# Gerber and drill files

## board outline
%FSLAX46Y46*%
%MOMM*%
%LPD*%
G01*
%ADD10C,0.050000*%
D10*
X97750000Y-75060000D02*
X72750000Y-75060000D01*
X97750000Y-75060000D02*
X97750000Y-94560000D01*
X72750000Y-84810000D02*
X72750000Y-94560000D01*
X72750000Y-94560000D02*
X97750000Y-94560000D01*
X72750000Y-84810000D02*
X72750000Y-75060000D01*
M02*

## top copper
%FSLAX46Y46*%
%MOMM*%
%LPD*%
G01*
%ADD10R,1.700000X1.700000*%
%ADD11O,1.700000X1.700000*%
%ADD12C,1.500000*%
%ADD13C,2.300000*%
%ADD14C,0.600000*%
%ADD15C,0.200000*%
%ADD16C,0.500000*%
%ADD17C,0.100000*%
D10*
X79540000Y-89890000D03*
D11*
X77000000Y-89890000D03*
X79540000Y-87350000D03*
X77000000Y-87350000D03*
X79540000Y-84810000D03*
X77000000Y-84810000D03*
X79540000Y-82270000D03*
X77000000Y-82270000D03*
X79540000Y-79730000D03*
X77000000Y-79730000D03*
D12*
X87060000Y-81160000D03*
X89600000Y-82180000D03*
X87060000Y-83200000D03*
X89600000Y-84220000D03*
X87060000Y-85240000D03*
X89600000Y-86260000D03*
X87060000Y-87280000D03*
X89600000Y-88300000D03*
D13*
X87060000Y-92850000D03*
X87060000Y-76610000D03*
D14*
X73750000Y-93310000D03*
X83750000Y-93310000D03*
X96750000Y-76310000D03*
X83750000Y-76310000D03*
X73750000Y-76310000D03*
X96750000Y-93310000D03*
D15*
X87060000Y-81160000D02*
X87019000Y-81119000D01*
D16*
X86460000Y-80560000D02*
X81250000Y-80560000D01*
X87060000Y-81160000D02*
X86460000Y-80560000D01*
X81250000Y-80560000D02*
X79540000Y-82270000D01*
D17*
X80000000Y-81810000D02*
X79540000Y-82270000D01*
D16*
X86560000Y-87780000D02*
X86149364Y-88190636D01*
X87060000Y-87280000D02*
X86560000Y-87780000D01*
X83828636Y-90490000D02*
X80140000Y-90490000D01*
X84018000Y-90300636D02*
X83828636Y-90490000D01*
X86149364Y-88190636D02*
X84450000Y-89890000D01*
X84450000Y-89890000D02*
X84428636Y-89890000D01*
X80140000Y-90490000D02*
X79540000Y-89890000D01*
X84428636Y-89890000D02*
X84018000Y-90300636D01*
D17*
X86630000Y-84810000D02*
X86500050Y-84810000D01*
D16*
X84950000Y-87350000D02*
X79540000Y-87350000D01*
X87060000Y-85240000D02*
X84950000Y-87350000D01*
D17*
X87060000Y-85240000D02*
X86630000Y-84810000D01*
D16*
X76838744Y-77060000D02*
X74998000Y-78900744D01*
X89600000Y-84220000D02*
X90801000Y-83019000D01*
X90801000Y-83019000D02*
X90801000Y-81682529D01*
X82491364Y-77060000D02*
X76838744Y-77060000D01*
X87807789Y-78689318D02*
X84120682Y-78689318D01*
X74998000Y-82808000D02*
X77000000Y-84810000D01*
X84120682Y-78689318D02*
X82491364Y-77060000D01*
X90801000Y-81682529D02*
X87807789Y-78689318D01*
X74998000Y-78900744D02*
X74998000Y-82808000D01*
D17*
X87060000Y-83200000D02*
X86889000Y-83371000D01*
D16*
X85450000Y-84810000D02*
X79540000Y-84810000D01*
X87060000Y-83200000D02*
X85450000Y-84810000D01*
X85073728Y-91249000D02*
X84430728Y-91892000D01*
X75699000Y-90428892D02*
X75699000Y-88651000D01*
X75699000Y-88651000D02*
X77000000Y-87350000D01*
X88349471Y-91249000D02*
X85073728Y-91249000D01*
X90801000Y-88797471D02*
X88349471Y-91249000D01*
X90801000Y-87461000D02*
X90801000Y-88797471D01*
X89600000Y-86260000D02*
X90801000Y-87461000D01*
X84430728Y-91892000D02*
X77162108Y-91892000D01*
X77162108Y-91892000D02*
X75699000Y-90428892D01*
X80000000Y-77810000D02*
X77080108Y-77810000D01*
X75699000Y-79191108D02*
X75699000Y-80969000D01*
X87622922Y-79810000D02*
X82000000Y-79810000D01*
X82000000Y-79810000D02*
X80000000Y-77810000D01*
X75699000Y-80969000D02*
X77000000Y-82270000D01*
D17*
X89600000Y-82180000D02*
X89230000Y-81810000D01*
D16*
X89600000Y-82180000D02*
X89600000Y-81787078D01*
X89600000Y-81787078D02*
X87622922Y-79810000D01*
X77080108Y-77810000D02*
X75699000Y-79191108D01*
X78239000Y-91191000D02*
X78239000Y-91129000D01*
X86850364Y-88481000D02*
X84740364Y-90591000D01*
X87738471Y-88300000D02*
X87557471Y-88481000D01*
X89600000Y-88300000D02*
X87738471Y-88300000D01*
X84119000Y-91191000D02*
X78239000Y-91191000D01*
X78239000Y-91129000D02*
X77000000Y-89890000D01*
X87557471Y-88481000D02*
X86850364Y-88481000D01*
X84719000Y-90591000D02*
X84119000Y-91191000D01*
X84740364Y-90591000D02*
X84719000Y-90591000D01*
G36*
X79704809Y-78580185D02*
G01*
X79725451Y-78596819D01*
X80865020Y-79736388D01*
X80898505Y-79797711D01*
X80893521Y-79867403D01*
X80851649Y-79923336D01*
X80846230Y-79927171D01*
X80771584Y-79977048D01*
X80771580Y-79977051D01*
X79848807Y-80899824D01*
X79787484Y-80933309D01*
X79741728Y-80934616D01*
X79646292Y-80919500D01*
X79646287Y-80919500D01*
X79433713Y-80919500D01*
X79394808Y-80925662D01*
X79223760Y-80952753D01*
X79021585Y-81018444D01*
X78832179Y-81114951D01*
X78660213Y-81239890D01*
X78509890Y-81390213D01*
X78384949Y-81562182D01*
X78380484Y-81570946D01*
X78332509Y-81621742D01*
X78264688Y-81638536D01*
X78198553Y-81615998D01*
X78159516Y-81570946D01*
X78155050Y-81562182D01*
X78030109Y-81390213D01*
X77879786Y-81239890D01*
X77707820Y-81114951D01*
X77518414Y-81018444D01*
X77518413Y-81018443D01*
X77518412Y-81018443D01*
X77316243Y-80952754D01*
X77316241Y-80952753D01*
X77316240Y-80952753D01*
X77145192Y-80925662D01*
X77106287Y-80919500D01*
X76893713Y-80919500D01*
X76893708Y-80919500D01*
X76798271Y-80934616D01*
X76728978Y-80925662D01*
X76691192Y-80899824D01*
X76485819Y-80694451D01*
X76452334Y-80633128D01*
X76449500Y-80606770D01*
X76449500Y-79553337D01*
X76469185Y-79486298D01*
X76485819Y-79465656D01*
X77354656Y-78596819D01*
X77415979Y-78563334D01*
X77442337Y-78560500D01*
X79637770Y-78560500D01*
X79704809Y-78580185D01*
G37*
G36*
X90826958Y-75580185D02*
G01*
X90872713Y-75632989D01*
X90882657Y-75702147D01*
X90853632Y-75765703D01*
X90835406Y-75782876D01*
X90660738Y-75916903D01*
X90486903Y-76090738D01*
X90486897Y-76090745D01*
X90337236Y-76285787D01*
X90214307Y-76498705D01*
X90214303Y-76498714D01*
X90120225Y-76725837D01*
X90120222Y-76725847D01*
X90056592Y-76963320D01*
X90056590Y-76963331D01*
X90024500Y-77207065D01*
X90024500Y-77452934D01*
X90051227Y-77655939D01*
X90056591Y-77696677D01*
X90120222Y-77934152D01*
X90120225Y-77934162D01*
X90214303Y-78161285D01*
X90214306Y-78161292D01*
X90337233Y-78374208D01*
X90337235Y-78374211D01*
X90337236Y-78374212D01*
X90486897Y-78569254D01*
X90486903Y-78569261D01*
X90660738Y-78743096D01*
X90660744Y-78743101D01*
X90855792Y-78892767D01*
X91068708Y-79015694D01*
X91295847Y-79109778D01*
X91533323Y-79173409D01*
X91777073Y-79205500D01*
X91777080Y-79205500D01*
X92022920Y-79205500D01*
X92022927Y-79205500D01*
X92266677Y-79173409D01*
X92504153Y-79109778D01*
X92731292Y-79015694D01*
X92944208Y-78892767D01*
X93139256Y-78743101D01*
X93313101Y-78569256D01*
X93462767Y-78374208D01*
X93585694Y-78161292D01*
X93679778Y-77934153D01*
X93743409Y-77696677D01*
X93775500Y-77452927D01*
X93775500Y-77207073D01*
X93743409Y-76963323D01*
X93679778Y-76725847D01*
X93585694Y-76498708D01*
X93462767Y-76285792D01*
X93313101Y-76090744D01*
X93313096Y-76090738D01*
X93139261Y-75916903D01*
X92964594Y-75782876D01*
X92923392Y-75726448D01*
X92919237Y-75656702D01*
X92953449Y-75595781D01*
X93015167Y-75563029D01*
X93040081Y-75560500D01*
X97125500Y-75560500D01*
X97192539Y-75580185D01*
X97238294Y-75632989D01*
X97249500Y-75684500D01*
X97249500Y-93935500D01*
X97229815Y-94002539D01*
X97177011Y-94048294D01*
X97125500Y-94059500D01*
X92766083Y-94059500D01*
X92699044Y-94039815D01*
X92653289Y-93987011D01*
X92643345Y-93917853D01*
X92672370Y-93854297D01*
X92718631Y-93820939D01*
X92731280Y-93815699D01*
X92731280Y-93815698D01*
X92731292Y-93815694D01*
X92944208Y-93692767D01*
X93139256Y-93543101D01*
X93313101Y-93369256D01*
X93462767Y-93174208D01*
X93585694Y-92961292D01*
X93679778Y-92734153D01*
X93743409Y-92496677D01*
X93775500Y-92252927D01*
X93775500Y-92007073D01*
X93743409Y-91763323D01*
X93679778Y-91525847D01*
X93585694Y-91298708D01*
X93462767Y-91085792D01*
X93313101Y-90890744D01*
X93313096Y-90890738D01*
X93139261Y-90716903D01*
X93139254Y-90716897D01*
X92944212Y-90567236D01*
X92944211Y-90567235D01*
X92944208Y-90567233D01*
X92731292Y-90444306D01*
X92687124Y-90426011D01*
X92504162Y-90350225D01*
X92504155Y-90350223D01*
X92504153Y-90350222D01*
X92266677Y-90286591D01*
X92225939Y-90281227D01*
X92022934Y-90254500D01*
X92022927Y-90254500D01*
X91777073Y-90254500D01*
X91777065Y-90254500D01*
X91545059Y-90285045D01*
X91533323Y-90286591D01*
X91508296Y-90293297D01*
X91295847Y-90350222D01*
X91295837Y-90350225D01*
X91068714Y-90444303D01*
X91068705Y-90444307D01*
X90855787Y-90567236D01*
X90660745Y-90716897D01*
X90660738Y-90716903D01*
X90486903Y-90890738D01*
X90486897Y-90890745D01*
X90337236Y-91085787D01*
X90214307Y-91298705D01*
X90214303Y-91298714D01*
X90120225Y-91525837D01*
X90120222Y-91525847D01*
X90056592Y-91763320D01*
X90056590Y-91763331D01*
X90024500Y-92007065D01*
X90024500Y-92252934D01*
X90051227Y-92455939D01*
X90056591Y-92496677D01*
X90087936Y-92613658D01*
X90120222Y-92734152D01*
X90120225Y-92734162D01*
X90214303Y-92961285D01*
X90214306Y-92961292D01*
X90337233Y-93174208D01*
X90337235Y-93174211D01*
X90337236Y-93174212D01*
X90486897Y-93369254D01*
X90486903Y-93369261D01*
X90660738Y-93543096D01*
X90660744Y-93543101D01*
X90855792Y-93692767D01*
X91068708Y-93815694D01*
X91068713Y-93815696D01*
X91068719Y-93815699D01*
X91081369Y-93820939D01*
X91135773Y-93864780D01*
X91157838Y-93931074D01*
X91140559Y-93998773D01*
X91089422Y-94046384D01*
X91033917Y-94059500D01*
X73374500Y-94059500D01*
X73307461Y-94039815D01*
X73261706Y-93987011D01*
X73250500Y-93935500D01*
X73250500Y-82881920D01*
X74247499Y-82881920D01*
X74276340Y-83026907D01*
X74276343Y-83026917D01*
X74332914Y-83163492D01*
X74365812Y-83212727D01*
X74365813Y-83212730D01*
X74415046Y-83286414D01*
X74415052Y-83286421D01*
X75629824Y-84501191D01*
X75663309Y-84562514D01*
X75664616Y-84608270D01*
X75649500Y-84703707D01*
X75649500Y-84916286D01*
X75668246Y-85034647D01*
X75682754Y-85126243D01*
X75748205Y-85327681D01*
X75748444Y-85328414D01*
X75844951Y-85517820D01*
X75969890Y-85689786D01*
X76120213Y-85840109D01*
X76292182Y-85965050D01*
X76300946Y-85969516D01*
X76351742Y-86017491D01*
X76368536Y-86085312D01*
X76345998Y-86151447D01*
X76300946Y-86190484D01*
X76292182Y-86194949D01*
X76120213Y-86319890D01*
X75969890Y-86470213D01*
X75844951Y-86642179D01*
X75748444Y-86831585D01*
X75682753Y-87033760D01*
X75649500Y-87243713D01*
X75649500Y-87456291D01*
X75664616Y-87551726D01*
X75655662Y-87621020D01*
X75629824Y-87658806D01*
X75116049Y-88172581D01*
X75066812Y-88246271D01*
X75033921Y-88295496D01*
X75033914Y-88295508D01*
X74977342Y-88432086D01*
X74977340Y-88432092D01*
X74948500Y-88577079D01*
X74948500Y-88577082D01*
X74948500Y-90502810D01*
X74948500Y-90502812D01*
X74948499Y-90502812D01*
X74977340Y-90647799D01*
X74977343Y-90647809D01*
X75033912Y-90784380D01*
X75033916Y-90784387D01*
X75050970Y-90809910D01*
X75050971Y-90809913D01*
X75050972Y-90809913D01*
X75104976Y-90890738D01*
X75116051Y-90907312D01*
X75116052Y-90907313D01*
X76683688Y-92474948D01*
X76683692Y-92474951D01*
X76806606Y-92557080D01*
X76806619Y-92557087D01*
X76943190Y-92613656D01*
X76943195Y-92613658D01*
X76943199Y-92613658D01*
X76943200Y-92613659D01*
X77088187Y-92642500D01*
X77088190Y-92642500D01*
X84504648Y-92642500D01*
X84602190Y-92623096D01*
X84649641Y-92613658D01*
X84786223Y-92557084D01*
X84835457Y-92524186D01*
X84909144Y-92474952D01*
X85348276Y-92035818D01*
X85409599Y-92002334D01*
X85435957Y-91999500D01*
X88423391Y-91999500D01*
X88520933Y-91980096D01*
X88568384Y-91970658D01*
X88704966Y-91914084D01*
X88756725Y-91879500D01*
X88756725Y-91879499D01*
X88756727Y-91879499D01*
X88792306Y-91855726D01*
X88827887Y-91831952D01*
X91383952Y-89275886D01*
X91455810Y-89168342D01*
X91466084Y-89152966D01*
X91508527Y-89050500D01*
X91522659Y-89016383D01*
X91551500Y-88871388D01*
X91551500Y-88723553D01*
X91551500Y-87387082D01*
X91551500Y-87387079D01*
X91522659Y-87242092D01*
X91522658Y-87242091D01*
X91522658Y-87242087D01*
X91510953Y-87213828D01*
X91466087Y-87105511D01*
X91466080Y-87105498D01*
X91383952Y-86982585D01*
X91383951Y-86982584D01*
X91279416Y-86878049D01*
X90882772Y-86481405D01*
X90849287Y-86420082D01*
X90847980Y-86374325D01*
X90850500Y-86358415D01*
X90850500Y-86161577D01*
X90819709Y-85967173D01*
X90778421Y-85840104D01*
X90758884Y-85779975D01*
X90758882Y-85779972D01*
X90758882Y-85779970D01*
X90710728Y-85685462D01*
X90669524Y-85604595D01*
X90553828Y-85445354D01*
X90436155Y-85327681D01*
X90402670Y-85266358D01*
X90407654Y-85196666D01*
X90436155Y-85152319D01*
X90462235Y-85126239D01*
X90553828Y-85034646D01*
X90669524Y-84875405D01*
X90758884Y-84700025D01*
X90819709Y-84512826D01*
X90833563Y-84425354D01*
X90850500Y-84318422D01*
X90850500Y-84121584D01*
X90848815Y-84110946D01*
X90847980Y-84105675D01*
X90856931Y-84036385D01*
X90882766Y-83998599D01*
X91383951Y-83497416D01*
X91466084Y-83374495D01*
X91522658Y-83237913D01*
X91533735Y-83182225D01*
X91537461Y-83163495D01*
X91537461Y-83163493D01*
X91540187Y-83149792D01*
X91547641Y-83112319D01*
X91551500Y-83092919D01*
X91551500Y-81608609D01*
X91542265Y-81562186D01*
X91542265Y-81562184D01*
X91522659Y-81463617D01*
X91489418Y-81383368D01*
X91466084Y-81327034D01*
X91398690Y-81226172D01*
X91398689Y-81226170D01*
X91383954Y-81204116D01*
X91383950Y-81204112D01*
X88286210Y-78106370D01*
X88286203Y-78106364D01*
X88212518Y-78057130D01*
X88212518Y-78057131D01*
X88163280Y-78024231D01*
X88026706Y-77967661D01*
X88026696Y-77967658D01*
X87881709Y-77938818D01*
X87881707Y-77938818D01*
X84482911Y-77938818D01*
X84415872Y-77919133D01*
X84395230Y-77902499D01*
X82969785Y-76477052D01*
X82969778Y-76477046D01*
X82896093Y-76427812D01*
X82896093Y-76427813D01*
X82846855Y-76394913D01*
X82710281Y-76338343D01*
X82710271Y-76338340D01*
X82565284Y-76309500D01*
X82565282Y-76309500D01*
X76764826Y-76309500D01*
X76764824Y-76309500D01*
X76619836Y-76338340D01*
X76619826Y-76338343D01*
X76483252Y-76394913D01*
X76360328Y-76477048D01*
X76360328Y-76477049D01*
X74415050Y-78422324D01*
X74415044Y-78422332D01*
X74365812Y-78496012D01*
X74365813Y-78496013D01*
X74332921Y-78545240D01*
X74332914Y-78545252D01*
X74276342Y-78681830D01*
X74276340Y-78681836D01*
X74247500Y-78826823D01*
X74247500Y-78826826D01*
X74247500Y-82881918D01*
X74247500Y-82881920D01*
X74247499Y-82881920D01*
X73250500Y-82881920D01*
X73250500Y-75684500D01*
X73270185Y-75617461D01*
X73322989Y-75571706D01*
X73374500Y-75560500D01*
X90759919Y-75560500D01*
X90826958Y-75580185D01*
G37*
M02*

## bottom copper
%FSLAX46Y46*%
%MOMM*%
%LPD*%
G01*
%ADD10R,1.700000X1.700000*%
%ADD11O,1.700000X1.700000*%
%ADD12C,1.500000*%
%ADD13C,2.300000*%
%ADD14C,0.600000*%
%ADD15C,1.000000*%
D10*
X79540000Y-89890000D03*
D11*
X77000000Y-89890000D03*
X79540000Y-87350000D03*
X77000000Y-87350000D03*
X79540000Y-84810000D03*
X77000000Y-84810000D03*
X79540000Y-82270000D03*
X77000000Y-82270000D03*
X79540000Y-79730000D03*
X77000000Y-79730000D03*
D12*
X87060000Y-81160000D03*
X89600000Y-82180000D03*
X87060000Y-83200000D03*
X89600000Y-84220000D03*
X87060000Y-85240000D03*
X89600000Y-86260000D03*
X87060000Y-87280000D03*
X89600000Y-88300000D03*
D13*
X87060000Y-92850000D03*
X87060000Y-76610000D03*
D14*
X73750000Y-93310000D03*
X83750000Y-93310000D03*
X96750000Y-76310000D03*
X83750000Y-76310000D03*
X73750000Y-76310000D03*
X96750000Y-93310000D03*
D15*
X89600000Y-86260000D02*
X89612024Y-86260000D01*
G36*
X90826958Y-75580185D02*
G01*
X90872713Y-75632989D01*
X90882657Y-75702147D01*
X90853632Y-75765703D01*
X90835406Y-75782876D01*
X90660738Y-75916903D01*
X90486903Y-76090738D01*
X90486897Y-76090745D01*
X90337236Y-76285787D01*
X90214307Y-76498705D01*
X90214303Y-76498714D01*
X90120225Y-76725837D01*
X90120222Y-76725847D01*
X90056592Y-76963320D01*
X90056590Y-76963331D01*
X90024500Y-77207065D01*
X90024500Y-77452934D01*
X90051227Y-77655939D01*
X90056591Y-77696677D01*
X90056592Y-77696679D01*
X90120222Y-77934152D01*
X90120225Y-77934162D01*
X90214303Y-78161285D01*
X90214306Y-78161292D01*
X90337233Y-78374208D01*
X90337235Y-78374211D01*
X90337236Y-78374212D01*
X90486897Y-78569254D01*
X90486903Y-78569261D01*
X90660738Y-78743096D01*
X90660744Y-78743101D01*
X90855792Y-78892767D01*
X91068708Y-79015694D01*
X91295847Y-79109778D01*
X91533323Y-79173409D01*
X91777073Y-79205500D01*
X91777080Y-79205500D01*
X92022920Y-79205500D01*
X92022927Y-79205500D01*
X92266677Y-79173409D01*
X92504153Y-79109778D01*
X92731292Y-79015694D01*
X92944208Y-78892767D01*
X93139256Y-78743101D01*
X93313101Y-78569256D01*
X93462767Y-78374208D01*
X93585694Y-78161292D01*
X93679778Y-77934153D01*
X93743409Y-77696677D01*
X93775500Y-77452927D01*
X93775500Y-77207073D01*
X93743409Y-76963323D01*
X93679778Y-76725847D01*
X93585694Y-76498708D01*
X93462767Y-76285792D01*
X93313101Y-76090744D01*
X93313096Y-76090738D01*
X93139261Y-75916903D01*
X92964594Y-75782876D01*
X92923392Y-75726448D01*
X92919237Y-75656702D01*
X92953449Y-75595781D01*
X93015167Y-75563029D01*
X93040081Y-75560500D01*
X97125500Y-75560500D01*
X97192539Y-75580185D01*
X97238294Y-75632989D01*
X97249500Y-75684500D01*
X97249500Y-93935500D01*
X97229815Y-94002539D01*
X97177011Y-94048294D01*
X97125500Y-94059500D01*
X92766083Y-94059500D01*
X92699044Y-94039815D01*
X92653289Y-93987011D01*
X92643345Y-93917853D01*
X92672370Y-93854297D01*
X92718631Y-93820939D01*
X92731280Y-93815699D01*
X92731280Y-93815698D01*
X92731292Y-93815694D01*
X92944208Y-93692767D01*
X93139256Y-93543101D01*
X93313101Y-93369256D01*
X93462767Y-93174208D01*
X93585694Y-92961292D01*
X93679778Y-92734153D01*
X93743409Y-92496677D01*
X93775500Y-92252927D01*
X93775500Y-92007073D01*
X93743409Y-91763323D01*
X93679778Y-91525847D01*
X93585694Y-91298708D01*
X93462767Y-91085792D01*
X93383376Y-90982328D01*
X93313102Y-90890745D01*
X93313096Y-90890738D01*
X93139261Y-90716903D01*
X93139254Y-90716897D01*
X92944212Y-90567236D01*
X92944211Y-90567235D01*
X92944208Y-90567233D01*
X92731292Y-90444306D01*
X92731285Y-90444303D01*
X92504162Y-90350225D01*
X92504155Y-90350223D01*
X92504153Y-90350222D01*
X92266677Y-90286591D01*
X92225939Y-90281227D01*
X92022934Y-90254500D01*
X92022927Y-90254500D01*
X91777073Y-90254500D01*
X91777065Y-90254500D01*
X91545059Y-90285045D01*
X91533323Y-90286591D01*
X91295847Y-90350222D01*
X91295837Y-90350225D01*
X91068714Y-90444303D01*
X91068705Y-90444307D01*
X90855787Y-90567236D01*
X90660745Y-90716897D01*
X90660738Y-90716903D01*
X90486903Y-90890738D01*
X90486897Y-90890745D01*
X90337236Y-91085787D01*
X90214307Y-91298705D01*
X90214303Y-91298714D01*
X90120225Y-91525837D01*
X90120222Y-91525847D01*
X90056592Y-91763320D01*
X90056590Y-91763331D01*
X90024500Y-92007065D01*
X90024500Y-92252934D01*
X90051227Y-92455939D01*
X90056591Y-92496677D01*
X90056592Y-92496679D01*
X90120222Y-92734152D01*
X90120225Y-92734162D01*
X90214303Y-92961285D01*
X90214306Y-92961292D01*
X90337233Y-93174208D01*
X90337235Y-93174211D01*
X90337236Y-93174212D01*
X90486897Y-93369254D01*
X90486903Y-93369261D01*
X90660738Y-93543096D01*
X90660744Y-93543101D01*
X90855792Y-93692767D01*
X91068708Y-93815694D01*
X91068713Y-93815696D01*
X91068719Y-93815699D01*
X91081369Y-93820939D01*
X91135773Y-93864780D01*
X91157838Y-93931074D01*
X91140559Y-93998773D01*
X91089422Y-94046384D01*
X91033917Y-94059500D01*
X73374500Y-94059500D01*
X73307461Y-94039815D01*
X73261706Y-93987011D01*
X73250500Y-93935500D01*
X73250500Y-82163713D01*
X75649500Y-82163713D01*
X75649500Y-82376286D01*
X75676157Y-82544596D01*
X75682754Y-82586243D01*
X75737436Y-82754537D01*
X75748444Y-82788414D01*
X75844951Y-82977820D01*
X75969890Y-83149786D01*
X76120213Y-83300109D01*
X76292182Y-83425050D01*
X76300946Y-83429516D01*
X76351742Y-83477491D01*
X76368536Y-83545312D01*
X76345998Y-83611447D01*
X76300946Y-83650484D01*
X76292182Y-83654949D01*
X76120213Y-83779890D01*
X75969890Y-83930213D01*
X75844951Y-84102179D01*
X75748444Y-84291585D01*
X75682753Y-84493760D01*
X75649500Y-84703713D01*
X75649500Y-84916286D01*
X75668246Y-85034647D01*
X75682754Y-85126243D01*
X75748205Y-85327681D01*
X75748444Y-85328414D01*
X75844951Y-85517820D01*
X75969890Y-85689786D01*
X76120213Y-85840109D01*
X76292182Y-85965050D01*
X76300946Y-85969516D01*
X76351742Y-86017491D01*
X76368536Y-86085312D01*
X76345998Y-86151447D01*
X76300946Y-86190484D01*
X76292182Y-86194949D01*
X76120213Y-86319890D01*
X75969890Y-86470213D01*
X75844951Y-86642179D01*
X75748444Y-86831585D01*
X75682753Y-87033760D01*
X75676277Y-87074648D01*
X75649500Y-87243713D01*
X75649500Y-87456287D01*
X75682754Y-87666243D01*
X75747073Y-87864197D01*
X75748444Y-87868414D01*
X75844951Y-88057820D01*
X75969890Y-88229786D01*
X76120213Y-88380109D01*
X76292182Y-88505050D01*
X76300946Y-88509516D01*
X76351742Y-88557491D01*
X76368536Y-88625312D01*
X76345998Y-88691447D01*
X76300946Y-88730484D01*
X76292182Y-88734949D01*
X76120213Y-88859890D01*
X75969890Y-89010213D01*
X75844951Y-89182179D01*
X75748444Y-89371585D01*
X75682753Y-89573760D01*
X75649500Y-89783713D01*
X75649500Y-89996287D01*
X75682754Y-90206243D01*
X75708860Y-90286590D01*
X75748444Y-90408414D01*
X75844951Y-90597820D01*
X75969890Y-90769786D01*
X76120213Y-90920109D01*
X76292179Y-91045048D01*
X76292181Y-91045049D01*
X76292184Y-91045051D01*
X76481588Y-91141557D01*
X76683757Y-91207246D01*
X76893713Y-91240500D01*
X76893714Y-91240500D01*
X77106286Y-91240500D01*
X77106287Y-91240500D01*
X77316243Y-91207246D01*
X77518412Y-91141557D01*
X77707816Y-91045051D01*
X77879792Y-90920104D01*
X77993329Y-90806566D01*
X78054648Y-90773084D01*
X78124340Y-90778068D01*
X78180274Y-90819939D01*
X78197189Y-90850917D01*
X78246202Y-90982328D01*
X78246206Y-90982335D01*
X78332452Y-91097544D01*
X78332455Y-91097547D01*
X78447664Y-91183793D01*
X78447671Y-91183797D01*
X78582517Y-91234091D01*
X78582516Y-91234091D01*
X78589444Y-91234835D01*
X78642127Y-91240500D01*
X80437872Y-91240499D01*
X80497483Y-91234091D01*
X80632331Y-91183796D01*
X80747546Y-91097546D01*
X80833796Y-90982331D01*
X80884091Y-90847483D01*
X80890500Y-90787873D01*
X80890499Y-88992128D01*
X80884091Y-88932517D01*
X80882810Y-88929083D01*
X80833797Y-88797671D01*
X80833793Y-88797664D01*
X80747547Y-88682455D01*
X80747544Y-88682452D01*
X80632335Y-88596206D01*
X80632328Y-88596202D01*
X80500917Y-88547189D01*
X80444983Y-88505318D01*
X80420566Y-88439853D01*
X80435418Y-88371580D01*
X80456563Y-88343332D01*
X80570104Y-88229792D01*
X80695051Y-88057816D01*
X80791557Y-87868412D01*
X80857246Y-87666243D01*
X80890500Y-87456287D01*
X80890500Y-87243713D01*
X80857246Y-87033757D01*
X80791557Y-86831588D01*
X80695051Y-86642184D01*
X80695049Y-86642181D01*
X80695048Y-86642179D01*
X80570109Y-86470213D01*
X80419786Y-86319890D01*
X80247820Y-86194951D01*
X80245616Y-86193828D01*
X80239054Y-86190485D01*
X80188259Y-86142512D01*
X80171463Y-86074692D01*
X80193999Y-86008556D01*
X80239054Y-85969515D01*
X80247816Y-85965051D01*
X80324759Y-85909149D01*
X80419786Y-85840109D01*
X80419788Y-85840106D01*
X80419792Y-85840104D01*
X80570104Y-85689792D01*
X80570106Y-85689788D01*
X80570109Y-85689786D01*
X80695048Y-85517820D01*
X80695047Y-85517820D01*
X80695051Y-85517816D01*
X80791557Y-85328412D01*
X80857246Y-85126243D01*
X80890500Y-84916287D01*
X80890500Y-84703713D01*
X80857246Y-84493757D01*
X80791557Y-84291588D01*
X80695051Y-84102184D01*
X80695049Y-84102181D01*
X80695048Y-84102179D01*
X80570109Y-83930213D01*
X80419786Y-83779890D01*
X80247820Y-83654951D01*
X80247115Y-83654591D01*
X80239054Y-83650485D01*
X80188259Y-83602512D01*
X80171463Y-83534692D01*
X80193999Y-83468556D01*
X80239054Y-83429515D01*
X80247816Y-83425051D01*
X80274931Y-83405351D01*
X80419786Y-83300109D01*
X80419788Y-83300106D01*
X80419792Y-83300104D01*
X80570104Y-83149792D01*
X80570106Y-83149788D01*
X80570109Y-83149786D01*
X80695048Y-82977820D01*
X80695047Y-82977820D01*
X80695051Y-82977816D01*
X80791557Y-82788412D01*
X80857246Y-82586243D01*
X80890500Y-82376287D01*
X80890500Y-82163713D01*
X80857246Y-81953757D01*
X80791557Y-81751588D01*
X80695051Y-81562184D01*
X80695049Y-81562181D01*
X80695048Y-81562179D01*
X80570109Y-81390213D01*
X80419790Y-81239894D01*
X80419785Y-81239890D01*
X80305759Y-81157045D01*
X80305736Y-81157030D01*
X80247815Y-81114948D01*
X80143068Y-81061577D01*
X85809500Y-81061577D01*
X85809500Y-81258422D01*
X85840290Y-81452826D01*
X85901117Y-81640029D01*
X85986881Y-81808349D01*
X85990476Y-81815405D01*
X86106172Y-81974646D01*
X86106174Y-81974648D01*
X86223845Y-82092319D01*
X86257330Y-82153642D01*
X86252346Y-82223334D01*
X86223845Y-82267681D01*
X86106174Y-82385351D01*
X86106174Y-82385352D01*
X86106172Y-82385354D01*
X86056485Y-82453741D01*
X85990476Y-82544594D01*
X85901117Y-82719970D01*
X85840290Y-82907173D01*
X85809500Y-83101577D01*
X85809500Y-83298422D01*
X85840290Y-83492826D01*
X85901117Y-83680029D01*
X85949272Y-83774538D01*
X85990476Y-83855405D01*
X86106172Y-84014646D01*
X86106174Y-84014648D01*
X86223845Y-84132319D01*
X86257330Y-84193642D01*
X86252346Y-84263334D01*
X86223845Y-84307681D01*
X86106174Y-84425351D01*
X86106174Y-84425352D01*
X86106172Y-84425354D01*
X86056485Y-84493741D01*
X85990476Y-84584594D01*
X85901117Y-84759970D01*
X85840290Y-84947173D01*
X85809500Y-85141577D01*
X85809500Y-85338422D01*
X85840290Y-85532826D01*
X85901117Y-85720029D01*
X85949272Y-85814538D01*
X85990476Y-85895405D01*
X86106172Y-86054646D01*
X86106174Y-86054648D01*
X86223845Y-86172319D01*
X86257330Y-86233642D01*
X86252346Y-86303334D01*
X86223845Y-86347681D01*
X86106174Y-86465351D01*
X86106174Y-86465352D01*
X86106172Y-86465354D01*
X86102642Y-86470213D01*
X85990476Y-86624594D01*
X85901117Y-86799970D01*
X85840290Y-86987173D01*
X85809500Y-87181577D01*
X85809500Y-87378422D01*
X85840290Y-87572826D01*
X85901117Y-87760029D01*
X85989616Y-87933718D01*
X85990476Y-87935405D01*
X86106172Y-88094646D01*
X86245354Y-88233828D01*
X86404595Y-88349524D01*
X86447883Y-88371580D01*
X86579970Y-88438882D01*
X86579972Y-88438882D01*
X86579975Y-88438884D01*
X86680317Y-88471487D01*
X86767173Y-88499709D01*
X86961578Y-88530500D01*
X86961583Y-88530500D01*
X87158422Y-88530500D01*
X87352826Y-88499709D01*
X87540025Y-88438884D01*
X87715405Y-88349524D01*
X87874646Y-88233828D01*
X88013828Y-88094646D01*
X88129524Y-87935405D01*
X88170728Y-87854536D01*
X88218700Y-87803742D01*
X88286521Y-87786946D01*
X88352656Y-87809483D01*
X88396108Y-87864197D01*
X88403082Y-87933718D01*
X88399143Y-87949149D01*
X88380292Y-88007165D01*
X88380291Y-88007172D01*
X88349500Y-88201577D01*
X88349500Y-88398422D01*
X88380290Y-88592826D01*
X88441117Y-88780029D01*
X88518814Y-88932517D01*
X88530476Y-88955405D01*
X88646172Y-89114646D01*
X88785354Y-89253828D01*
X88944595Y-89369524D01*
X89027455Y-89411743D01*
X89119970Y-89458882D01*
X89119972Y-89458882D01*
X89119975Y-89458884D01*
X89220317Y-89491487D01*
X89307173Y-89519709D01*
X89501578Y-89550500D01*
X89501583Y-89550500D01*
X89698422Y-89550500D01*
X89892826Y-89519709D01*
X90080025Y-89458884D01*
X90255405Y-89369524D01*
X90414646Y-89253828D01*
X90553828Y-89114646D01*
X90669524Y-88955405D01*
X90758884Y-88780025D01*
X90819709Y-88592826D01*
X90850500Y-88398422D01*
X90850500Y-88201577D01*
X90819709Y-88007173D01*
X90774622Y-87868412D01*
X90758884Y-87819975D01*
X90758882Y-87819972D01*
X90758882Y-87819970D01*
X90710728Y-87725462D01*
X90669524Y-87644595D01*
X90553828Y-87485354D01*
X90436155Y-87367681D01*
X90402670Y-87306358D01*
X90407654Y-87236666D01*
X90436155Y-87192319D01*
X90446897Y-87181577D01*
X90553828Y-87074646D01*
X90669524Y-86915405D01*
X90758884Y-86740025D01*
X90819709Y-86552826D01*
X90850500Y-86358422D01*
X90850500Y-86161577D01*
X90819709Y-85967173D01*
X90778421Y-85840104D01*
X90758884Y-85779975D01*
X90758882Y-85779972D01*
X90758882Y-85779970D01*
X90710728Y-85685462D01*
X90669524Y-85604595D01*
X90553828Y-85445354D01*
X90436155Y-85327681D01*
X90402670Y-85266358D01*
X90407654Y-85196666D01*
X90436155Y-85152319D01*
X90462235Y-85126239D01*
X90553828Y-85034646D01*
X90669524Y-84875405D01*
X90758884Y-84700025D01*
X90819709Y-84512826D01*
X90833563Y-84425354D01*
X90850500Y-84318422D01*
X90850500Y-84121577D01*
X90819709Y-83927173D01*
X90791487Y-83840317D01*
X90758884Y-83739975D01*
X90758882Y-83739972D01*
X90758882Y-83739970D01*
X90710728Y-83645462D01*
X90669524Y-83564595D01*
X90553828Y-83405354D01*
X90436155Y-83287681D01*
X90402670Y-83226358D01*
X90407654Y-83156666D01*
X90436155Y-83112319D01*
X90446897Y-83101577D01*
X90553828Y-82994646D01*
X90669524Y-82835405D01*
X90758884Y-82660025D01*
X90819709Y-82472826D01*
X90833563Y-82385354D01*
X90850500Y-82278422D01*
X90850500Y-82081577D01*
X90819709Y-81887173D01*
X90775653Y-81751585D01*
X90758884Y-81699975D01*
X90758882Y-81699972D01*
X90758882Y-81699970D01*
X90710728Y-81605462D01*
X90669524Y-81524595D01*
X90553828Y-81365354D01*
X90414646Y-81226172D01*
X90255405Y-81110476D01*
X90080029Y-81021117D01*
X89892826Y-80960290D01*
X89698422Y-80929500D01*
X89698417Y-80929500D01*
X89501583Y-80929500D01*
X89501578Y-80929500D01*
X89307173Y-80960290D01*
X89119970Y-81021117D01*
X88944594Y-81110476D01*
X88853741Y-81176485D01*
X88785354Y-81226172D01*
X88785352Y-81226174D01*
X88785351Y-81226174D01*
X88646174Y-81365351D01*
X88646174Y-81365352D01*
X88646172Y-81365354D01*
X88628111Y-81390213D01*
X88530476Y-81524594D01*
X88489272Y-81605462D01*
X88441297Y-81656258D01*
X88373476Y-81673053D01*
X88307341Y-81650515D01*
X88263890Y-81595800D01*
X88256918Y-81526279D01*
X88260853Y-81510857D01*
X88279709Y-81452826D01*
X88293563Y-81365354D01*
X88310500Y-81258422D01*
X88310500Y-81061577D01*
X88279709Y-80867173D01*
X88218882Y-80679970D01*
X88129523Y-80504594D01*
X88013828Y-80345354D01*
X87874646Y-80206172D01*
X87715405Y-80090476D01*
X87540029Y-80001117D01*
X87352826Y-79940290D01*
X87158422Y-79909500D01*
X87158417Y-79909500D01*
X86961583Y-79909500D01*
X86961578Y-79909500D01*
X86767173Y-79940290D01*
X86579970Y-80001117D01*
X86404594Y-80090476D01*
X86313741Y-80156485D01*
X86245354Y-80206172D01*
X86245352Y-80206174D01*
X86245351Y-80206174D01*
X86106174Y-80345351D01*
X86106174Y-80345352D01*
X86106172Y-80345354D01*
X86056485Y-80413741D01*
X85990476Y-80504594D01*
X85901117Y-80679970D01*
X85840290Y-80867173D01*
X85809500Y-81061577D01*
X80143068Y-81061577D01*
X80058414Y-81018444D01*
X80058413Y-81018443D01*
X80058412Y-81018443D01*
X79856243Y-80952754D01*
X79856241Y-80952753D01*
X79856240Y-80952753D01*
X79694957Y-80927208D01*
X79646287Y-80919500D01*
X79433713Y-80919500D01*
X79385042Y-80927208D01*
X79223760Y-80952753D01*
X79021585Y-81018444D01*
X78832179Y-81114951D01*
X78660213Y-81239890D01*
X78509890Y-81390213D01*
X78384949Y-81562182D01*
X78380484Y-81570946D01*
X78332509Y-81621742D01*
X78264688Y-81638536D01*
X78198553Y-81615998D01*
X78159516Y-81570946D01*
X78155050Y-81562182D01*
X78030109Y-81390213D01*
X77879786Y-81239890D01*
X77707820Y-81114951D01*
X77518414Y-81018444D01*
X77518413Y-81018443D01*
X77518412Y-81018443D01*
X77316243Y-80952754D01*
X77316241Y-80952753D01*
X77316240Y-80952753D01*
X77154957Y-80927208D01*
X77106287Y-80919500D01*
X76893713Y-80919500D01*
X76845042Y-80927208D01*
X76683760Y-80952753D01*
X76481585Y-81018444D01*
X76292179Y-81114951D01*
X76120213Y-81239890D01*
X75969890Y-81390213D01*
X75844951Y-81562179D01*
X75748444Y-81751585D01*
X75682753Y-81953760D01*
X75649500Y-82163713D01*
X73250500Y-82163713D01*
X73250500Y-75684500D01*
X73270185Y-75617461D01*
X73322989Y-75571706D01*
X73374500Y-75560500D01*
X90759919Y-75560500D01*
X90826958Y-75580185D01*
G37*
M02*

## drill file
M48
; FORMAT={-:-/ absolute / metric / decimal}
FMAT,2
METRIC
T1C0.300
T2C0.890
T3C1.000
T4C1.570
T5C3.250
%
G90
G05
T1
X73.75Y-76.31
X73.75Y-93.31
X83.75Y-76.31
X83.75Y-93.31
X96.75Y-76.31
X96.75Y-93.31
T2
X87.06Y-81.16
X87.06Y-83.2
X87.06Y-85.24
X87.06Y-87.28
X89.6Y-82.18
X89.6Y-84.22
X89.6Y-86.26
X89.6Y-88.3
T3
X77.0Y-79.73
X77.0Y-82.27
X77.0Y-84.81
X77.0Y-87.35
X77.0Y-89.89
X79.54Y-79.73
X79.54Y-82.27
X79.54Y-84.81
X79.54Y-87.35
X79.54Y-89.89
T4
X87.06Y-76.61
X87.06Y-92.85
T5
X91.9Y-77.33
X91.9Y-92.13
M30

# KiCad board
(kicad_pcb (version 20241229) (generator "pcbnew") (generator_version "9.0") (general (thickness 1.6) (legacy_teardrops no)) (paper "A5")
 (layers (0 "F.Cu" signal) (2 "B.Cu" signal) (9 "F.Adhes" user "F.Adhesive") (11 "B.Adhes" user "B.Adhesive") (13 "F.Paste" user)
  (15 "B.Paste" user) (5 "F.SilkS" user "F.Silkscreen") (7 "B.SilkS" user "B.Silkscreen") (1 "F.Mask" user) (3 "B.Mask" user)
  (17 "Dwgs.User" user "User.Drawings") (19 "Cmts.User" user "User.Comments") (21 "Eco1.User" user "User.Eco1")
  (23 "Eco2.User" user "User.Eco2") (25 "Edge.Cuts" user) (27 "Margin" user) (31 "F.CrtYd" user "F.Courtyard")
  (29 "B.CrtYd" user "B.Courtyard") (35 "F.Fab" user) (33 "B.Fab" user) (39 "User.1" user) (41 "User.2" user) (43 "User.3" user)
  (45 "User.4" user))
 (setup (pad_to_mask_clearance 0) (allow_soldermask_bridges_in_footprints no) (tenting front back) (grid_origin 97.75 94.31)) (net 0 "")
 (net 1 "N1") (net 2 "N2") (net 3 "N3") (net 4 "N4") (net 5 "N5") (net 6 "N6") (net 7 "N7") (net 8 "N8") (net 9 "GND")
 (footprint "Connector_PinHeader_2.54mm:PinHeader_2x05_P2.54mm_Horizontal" (layer "F.Cu") (at 79.54 89.89 180)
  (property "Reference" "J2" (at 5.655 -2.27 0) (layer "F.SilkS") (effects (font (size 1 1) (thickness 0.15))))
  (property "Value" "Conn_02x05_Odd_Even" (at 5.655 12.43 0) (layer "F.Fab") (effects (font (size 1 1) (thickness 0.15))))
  (pad "1" thru_hole rect (at 0 0 180) (size 1.7 1.7) (drill 1) (layers "*.Cu" "*.Mask") (remove_unused_layers no) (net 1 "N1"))
  (pad "2" thru_hole oval (at 2.54 0 180) (size 1.7 1.7) (drill 1) (layers "*.Cu" "*.Mask") (remove_unused_layers no) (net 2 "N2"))
  (pad "3" thru_hole oval (at 0 2.54 180) (size 1.7 1.7) (drill 1) (layers "*.Cu" "*.Mask") (remove_unused_layers no) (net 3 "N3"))
  (pad "4" thru_hole oval (at 2.54 2.54 180) (size 1.7 1.7) (drill 1) (layers "*.Cu" "*.Mask") (remove_unused_layers no) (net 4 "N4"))
  (pad "5" thru_hole oval (at 0 5.08 180) (size 1.7 1.7) (drill 1) (layers "*.Cu" "*.Mask") (remove_unused_layers no) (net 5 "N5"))
  (pad "6" thru_hole oval (at 2.54 5.08 180) (size 1.7 1.7) (drill 1) (layers "*.Cu" "*.Mask") (remove_unused_layers no) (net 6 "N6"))
  (pad "7" thru_hole oval (at 0 7.62 180) (size 1.7 1.7) (drill 1) (layers "*.Cu" "*.Mask") (remove_unused_layers no) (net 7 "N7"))
  (pad "8" thru_hole oval (at 2.54 7.62 180) (size 1.7 1.7) (drill 1) (layers "*.Cu" "*.Mask") (remove_unused_layers no) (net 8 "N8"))
  (pad "9" thru_hole oval (at 0 10.16 180) (size 1.7 1.7) (drill 1) (layers "*.Cu" "*.Mask") (remove_unused_layers no) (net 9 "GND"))
  (pad "10" thru_hole oval (at 2.54 10.16 180) (size 1.7 1.7) (drill 1) (layers "*.Cu" "*.Mask") (remove_unused_layers no) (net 9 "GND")))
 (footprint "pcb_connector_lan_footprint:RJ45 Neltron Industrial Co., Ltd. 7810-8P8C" (layer "F.Cu") (at 91.9 77.33 90)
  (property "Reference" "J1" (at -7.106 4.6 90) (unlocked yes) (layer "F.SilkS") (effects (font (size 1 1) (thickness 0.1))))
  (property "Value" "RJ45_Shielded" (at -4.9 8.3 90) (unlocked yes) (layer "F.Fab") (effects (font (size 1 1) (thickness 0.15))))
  (pad "" np_thru_hole circle (at -14.8 0 90) (size 3.25 3.25) (drill 3.25) (layers "*.Cu" "*.Mask"))
  (pad "" np_thru_hole circle (at 0 0 90) (size 3.25 3.25) (drill 3.25) (layers "*.Cu" "*.Mask"))
  (pad "1" thru_hole circle (at -3.83 -4.84 90) (size 1.5 1.5) (drill 0.89) (layers "*.Cu" "*.Mask") (remove_unused_layers no) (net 7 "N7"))
  (pad "2" thru_hole circle (at -4.85 -2.3 90) (size 1.5 1.5) (drill 0.89) (layers "*.Cu" "*.Mask") (remove_unused_layers no) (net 8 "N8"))
  (pad "3" thru_hole circle (at -5.87 -4.84 90) (size 1.5 1.5) (drill 0.89) (layers "*.Cu" "*.Mask") (remove_unused_layers no) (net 5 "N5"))
  (pad "4" thru_hole circle (at -6.89 -2.3 90) (size 1.5 1.5) (drill 0.89) (layers "*.Cu" "*.Mask") (remove_unused_layers no) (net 6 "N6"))
  (pad "5" thru_hole circle (at -7.91 -4.84 90) (size 1.5 1.5) (drill 0.89) (layers "*.Cu" "*.Mask") (remove_unused_layers no) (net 3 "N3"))
  (pad "6" thru_hole circle (at -8.93 -2.3 90) (size 1.5 1.5) (drill 0.89) (layers "*.Cu" "*.Mask") (remove_unused_layers no) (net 4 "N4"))
  (pad "7" thru_hole circle (at -9.95 -4.84 90) (size 1.5 1.5) (drill 0.89) (layers "*.Cu" "*.Mask") (remove_unused_layers no) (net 1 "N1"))
  (pad "8" thru_hole circle (at -10.97 -2.3 90) (size 1.5 1.5) (drill 0.89) (layers "*.Cu" "*.Mask") (remove_unused_layers no) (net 2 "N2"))
  (pad "SH" thru_hole circle (at -15.52 -4.84 90) (size 2.3 2.3) (drill 1.57) (layers "*.Cu" "*.Mask") (remove_unused_layers no)
   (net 9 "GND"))
  (pad "SH" thru_hole circle (at 0.72 -4.84 90) (size 2.3 2.3) (drill 1.57) (layers "*.Cu" "*.Mask") (remove_unused_layers no) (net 9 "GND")))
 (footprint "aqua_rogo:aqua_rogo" (layer "B.Cu") (at 93.75 85.06 -90)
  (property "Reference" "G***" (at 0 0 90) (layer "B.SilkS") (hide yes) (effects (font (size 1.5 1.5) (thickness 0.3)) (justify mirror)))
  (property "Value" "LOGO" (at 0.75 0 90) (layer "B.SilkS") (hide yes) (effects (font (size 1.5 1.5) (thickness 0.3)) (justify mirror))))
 (gr_line (start 97.75 75.06) (end 72.75 75.06) (stroke (width 0.05) (type default)) (layer "Edge.Cuts"))
 (gr_line (start 97.75 75.06) (end 97.75 94.56) (stroke (width 0.05) (type default)) (layer "Edge.Cuts"))
 (gr_line (start 72.75 84.81) (end 72.75 94.56) (stroke (width 0.05) (type default)) (layer "Edge.Cuts"))
 (gr_line (start 72.75 94.56) (end 97.75 94.56) (stroke (width 0.05) (type default)) (layer "Edge.Cuts"))
 (gr_line (start 72.75 84.81) (end 72.75 75.06) (stroke (width 0.05) (type default)) (layer "Edge.Cuts"))
 (via (at 73.75 93.31) (size 0.6) (drill 0.3) (layers "F.Cu" "B.Cu") (free yes) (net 9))
 (via (at 83.75 93.31) (size 0.6) (drill 0.3) (layers "F.Cu" "B.Cu") (free yes) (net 9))
 (via (at 96.75 76.31) (size 0.6) (drill 0.3) (layers "F.Cu" "B.Cu") (free yes) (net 9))
 (via (at 83.75 76.31) (size 0.6) (drill 0.3) (layers "F.Cu" "B.Cu") (free yes) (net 9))
 (via (at 73.75 76.31) (size 0.6) (drill 0.3) (layers "F.Cu" "B.Cu") (free yes) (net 9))
 (via (at 96.75 93.31) (size 0.6) (drill 0.3) (layers "F.Cu" "B.Cu") (free yes) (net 9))
 (segment (start 87.06 81.16) (end 87.019 81.119) (width 0.2) (layer "F.Cu") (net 7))
 (segment (start 86.46 80.56) (end 81.25 80.56) (width 0.5) (layer "F.Cu") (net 7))
 (segment (start 87.06 81.16) (end 86.46 80.56) (width 0.5) (layer "F.Cu") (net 7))
 (segment (start 81.25 80.56) (end 79.54 82.27) (width 0.5) (layer "F.Cu") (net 7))
 (segment (start 80 81.81) (end 79.54 82.27) (width 0.1) (layer "F.Cu") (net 7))
 (segment (start 86.56 87.78) (end 86.149364 88.190636) (width 0.5) (layer "F.Cu") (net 1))
 (segment (start 87.06 87.28) (end 86.56 87.78) (width 0.5) (layer "F.Cu") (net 1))
 (segment (start 83.828636 90.49) (end 80.14 90.49) (width 0.5) (layer "F.Cu") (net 1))
 (segment (start 84.018 90.300636) (end 83.828636 90.49) (width 0.5) (layer "F.Cu") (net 1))
 (segment (start 86.149364 88.190636) (end 84.45 89.89) (width 0.5) (layer "F.Cu") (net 1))
 (segment (start 84.45 89.89) (end 84.428636 89.89) (width 0.5) (layer "F.Cu") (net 1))
 (segment (start 80.14 90.49) (end 79.54 89.89) (width 0.5) (layer "F.Cu") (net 1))
 (segment (start 84.428636 89.89) (end 84.018 90.300636) (width 0.5) (layer "F.Cu") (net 1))
 (segment (start 86.63 84.81) (end 86.50005 84.81) (width 0.1) (layer "F.Cu") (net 3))
 (segment (start 84.95 87.35) (end 79.54 87.35) (width 0.5) (layer "F.Cu") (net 3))
 (segment (start 87.06 85.24) (end 84.95 87.35) (width 0.5) (layer "F.Cu") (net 3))
 (segment (start 87.06 85.24) (end 86.63 84.81) (width 0.1) (layer "F.Cu") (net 3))
 (segment (start 76.838744 77.06) (end 74.998 78.900744) (width 0.5) (layer "F.Cu") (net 6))
 (segment (start 89.6 84.22) (end 90.801 83.019) (width 0.5) (layer "F.Cu") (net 6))
 (segment (start 90.801 83.019) (end 90.801 81.682529) (width 0.5) (layer "F.Cu") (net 6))
 (segment (start 82.491364 77.06) (end 76.838744 77.06) (width 0.5) (layer "F.Cu") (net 6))
 (segment (start 87.807789 78.689318) (end 84.120682 78.689318) (width 0.5) (layer "F.Cu") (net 6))
 (segment (start 74.998 82.808) (end 77 84.81) (width 0.5) (layer "F.Cu") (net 6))
 (segment (start 84.120682 78.689318) (end 82.491364 77.06) (width 0.5) (layer "F.Cu") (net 6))
 (segment (start 90.801 81.682529) (end 87.807789 78.689318) (width 0.5) (layer "F.Cu") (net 6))
 (segment (start 74.998 78.900744) (end 74.998 82.808) (width 0.5) (layer "F.Cu") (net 6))
 (segment (start 87.06 83.2) (end 86.889 83.371) (width 0.1) (layer "F.Cu") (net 5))
 (segment (start 85.45 84.81) (end 79.54 84.81) (width 0.5) (layer "F.Cu") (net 5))
 (segment (start 87.06 83.2) (end 85.45 84.81) (width 0.5) (layer "F.Cu") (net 5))
 (segment (start 85.073728 91.249) (end 84.430728 91.892) (width 0.5) (layer "F.Cu") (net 4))
 (segment (start 75.699 90.428892) (end 75.699 88.651) (width 0.5) (layer "F.Cu") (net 4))
 (segment (start 75.699 88.651) (end 77 87.35) (width 0.5) (layer "F.Cu") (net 4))
 (segment (start 88.349471 91.249) (end 85.073728 91.249) (width 0.5) (layer "F.Cu") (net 4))
 (segment (start 90.801 88.797471) (end 88.349471 91.249) (width 0.5) (layer "F.Cu") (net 4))
 (segment (start 90.801 87.461) (end 90.801 88.797471) (width 0.5) (layer "F.Cu") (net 4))
 (segment (start 89.6 86.26) (end 90.801 87.461) (width 0.5) (layer "F.Cu") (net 4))
 (segment (start 84.430728 91.892) (end 77.162108 91.892) (width 0.5) (layer "F.Cu") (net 4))
 (segment (start 77.162108 91.892) (end 75.699 90.428892) (width 0.5) (layer "F.Cu") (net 4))
 (segment (start 89.6 86.26) (end 89.612024 86.26) (width 1) (layer "B.Cu") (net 4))
 (segment (start 80 77.81) (end 77.080108 77.81) (width 0.5) (layer "F.Cu") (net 8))
 (segment (start 75.699 79.191108) (end 75.699 80.969) (width 0.5) (layer "F.Cu") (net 8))
 (segment (start 87.622922 79.81) (end 82 79.81) (width 0.5) (layer "F.Cu") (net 8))
 (segment (start 82 79.81) (end 80 77.81) (width 0.5) (layer "F.Cu") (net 8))
 (segment (start 75.699 80.969) (end 77 82.27) (width 0.5) (layer "F.Cu") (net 8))
 (segment (start 89.6 82.18) (end 89.23 81.81) (width 0.1) (layer "F.Cu") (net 8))
 (segment (start 89.6 82.18) (end 89.6 81.787078) (width 0.5) (layer "F.Cu") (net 8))
 (segment (start 89.6 81.787078) (end 87.622922 79.81) (width 0.5) (layer "F.Cu") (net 8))
 (segment (start 77.080108 77.81) (end 75.699 79.191108) (width 0.5) (layer "F.Cu") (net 8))
 (segment (start 78.239 91.191) (end 78.239 91.129) (width 0.5) (layer "F.Cu") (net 2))
 (segment (start 86.850364 88.481) (end 84.740364 90.591) (width 0.5) (layer "F.Cu") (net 2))
 (segment (start 87.738471 88.3) (end 87.557471 88.481) (width 0.5) (layer "F.Cu") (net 2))
 (segment (start 89.6 88.3) (end 87.738471 88.3) (width 0.5) (layer "F.Cu") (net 2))
 (segment (start 84.119 91.191) (end 78.239 91.191) (width 0.5) (layer "F.Cu") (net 2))
 (segment (start 78.239 91.129) (end 77 89.89) (width 0.5) (layer "F.Cu") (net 2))
 (segment (start 87.557471 88.481) (end 86.850364 88.481) (width 0.5) (layer "F.Cu") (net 2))
 (segment (start 84.719 90.591) (end 84.119 91.191) (width 0.5) (layer "F.Cu") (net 2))
 (segment (start 84.740364 90.591) (end 84.719 90.591) (width 0.5) (layer "F.Cu") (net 2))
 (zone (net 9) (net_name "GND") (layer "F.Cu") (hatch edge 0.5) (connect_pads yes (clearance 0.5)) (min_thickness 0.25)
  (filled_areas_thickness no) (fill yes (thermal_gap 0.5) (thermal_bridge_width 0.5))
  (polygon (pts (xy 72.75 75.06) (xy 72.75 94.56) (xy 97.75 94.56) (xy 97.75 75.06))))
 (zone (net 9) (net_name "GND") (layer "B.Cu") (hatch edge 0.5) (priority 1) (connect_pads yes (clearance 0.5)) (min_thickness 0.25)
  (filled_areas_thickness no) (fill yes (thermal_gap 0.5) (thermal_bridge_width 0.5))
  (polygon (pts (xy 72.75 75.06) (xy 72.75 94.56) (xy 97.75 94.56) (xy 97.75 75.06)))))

